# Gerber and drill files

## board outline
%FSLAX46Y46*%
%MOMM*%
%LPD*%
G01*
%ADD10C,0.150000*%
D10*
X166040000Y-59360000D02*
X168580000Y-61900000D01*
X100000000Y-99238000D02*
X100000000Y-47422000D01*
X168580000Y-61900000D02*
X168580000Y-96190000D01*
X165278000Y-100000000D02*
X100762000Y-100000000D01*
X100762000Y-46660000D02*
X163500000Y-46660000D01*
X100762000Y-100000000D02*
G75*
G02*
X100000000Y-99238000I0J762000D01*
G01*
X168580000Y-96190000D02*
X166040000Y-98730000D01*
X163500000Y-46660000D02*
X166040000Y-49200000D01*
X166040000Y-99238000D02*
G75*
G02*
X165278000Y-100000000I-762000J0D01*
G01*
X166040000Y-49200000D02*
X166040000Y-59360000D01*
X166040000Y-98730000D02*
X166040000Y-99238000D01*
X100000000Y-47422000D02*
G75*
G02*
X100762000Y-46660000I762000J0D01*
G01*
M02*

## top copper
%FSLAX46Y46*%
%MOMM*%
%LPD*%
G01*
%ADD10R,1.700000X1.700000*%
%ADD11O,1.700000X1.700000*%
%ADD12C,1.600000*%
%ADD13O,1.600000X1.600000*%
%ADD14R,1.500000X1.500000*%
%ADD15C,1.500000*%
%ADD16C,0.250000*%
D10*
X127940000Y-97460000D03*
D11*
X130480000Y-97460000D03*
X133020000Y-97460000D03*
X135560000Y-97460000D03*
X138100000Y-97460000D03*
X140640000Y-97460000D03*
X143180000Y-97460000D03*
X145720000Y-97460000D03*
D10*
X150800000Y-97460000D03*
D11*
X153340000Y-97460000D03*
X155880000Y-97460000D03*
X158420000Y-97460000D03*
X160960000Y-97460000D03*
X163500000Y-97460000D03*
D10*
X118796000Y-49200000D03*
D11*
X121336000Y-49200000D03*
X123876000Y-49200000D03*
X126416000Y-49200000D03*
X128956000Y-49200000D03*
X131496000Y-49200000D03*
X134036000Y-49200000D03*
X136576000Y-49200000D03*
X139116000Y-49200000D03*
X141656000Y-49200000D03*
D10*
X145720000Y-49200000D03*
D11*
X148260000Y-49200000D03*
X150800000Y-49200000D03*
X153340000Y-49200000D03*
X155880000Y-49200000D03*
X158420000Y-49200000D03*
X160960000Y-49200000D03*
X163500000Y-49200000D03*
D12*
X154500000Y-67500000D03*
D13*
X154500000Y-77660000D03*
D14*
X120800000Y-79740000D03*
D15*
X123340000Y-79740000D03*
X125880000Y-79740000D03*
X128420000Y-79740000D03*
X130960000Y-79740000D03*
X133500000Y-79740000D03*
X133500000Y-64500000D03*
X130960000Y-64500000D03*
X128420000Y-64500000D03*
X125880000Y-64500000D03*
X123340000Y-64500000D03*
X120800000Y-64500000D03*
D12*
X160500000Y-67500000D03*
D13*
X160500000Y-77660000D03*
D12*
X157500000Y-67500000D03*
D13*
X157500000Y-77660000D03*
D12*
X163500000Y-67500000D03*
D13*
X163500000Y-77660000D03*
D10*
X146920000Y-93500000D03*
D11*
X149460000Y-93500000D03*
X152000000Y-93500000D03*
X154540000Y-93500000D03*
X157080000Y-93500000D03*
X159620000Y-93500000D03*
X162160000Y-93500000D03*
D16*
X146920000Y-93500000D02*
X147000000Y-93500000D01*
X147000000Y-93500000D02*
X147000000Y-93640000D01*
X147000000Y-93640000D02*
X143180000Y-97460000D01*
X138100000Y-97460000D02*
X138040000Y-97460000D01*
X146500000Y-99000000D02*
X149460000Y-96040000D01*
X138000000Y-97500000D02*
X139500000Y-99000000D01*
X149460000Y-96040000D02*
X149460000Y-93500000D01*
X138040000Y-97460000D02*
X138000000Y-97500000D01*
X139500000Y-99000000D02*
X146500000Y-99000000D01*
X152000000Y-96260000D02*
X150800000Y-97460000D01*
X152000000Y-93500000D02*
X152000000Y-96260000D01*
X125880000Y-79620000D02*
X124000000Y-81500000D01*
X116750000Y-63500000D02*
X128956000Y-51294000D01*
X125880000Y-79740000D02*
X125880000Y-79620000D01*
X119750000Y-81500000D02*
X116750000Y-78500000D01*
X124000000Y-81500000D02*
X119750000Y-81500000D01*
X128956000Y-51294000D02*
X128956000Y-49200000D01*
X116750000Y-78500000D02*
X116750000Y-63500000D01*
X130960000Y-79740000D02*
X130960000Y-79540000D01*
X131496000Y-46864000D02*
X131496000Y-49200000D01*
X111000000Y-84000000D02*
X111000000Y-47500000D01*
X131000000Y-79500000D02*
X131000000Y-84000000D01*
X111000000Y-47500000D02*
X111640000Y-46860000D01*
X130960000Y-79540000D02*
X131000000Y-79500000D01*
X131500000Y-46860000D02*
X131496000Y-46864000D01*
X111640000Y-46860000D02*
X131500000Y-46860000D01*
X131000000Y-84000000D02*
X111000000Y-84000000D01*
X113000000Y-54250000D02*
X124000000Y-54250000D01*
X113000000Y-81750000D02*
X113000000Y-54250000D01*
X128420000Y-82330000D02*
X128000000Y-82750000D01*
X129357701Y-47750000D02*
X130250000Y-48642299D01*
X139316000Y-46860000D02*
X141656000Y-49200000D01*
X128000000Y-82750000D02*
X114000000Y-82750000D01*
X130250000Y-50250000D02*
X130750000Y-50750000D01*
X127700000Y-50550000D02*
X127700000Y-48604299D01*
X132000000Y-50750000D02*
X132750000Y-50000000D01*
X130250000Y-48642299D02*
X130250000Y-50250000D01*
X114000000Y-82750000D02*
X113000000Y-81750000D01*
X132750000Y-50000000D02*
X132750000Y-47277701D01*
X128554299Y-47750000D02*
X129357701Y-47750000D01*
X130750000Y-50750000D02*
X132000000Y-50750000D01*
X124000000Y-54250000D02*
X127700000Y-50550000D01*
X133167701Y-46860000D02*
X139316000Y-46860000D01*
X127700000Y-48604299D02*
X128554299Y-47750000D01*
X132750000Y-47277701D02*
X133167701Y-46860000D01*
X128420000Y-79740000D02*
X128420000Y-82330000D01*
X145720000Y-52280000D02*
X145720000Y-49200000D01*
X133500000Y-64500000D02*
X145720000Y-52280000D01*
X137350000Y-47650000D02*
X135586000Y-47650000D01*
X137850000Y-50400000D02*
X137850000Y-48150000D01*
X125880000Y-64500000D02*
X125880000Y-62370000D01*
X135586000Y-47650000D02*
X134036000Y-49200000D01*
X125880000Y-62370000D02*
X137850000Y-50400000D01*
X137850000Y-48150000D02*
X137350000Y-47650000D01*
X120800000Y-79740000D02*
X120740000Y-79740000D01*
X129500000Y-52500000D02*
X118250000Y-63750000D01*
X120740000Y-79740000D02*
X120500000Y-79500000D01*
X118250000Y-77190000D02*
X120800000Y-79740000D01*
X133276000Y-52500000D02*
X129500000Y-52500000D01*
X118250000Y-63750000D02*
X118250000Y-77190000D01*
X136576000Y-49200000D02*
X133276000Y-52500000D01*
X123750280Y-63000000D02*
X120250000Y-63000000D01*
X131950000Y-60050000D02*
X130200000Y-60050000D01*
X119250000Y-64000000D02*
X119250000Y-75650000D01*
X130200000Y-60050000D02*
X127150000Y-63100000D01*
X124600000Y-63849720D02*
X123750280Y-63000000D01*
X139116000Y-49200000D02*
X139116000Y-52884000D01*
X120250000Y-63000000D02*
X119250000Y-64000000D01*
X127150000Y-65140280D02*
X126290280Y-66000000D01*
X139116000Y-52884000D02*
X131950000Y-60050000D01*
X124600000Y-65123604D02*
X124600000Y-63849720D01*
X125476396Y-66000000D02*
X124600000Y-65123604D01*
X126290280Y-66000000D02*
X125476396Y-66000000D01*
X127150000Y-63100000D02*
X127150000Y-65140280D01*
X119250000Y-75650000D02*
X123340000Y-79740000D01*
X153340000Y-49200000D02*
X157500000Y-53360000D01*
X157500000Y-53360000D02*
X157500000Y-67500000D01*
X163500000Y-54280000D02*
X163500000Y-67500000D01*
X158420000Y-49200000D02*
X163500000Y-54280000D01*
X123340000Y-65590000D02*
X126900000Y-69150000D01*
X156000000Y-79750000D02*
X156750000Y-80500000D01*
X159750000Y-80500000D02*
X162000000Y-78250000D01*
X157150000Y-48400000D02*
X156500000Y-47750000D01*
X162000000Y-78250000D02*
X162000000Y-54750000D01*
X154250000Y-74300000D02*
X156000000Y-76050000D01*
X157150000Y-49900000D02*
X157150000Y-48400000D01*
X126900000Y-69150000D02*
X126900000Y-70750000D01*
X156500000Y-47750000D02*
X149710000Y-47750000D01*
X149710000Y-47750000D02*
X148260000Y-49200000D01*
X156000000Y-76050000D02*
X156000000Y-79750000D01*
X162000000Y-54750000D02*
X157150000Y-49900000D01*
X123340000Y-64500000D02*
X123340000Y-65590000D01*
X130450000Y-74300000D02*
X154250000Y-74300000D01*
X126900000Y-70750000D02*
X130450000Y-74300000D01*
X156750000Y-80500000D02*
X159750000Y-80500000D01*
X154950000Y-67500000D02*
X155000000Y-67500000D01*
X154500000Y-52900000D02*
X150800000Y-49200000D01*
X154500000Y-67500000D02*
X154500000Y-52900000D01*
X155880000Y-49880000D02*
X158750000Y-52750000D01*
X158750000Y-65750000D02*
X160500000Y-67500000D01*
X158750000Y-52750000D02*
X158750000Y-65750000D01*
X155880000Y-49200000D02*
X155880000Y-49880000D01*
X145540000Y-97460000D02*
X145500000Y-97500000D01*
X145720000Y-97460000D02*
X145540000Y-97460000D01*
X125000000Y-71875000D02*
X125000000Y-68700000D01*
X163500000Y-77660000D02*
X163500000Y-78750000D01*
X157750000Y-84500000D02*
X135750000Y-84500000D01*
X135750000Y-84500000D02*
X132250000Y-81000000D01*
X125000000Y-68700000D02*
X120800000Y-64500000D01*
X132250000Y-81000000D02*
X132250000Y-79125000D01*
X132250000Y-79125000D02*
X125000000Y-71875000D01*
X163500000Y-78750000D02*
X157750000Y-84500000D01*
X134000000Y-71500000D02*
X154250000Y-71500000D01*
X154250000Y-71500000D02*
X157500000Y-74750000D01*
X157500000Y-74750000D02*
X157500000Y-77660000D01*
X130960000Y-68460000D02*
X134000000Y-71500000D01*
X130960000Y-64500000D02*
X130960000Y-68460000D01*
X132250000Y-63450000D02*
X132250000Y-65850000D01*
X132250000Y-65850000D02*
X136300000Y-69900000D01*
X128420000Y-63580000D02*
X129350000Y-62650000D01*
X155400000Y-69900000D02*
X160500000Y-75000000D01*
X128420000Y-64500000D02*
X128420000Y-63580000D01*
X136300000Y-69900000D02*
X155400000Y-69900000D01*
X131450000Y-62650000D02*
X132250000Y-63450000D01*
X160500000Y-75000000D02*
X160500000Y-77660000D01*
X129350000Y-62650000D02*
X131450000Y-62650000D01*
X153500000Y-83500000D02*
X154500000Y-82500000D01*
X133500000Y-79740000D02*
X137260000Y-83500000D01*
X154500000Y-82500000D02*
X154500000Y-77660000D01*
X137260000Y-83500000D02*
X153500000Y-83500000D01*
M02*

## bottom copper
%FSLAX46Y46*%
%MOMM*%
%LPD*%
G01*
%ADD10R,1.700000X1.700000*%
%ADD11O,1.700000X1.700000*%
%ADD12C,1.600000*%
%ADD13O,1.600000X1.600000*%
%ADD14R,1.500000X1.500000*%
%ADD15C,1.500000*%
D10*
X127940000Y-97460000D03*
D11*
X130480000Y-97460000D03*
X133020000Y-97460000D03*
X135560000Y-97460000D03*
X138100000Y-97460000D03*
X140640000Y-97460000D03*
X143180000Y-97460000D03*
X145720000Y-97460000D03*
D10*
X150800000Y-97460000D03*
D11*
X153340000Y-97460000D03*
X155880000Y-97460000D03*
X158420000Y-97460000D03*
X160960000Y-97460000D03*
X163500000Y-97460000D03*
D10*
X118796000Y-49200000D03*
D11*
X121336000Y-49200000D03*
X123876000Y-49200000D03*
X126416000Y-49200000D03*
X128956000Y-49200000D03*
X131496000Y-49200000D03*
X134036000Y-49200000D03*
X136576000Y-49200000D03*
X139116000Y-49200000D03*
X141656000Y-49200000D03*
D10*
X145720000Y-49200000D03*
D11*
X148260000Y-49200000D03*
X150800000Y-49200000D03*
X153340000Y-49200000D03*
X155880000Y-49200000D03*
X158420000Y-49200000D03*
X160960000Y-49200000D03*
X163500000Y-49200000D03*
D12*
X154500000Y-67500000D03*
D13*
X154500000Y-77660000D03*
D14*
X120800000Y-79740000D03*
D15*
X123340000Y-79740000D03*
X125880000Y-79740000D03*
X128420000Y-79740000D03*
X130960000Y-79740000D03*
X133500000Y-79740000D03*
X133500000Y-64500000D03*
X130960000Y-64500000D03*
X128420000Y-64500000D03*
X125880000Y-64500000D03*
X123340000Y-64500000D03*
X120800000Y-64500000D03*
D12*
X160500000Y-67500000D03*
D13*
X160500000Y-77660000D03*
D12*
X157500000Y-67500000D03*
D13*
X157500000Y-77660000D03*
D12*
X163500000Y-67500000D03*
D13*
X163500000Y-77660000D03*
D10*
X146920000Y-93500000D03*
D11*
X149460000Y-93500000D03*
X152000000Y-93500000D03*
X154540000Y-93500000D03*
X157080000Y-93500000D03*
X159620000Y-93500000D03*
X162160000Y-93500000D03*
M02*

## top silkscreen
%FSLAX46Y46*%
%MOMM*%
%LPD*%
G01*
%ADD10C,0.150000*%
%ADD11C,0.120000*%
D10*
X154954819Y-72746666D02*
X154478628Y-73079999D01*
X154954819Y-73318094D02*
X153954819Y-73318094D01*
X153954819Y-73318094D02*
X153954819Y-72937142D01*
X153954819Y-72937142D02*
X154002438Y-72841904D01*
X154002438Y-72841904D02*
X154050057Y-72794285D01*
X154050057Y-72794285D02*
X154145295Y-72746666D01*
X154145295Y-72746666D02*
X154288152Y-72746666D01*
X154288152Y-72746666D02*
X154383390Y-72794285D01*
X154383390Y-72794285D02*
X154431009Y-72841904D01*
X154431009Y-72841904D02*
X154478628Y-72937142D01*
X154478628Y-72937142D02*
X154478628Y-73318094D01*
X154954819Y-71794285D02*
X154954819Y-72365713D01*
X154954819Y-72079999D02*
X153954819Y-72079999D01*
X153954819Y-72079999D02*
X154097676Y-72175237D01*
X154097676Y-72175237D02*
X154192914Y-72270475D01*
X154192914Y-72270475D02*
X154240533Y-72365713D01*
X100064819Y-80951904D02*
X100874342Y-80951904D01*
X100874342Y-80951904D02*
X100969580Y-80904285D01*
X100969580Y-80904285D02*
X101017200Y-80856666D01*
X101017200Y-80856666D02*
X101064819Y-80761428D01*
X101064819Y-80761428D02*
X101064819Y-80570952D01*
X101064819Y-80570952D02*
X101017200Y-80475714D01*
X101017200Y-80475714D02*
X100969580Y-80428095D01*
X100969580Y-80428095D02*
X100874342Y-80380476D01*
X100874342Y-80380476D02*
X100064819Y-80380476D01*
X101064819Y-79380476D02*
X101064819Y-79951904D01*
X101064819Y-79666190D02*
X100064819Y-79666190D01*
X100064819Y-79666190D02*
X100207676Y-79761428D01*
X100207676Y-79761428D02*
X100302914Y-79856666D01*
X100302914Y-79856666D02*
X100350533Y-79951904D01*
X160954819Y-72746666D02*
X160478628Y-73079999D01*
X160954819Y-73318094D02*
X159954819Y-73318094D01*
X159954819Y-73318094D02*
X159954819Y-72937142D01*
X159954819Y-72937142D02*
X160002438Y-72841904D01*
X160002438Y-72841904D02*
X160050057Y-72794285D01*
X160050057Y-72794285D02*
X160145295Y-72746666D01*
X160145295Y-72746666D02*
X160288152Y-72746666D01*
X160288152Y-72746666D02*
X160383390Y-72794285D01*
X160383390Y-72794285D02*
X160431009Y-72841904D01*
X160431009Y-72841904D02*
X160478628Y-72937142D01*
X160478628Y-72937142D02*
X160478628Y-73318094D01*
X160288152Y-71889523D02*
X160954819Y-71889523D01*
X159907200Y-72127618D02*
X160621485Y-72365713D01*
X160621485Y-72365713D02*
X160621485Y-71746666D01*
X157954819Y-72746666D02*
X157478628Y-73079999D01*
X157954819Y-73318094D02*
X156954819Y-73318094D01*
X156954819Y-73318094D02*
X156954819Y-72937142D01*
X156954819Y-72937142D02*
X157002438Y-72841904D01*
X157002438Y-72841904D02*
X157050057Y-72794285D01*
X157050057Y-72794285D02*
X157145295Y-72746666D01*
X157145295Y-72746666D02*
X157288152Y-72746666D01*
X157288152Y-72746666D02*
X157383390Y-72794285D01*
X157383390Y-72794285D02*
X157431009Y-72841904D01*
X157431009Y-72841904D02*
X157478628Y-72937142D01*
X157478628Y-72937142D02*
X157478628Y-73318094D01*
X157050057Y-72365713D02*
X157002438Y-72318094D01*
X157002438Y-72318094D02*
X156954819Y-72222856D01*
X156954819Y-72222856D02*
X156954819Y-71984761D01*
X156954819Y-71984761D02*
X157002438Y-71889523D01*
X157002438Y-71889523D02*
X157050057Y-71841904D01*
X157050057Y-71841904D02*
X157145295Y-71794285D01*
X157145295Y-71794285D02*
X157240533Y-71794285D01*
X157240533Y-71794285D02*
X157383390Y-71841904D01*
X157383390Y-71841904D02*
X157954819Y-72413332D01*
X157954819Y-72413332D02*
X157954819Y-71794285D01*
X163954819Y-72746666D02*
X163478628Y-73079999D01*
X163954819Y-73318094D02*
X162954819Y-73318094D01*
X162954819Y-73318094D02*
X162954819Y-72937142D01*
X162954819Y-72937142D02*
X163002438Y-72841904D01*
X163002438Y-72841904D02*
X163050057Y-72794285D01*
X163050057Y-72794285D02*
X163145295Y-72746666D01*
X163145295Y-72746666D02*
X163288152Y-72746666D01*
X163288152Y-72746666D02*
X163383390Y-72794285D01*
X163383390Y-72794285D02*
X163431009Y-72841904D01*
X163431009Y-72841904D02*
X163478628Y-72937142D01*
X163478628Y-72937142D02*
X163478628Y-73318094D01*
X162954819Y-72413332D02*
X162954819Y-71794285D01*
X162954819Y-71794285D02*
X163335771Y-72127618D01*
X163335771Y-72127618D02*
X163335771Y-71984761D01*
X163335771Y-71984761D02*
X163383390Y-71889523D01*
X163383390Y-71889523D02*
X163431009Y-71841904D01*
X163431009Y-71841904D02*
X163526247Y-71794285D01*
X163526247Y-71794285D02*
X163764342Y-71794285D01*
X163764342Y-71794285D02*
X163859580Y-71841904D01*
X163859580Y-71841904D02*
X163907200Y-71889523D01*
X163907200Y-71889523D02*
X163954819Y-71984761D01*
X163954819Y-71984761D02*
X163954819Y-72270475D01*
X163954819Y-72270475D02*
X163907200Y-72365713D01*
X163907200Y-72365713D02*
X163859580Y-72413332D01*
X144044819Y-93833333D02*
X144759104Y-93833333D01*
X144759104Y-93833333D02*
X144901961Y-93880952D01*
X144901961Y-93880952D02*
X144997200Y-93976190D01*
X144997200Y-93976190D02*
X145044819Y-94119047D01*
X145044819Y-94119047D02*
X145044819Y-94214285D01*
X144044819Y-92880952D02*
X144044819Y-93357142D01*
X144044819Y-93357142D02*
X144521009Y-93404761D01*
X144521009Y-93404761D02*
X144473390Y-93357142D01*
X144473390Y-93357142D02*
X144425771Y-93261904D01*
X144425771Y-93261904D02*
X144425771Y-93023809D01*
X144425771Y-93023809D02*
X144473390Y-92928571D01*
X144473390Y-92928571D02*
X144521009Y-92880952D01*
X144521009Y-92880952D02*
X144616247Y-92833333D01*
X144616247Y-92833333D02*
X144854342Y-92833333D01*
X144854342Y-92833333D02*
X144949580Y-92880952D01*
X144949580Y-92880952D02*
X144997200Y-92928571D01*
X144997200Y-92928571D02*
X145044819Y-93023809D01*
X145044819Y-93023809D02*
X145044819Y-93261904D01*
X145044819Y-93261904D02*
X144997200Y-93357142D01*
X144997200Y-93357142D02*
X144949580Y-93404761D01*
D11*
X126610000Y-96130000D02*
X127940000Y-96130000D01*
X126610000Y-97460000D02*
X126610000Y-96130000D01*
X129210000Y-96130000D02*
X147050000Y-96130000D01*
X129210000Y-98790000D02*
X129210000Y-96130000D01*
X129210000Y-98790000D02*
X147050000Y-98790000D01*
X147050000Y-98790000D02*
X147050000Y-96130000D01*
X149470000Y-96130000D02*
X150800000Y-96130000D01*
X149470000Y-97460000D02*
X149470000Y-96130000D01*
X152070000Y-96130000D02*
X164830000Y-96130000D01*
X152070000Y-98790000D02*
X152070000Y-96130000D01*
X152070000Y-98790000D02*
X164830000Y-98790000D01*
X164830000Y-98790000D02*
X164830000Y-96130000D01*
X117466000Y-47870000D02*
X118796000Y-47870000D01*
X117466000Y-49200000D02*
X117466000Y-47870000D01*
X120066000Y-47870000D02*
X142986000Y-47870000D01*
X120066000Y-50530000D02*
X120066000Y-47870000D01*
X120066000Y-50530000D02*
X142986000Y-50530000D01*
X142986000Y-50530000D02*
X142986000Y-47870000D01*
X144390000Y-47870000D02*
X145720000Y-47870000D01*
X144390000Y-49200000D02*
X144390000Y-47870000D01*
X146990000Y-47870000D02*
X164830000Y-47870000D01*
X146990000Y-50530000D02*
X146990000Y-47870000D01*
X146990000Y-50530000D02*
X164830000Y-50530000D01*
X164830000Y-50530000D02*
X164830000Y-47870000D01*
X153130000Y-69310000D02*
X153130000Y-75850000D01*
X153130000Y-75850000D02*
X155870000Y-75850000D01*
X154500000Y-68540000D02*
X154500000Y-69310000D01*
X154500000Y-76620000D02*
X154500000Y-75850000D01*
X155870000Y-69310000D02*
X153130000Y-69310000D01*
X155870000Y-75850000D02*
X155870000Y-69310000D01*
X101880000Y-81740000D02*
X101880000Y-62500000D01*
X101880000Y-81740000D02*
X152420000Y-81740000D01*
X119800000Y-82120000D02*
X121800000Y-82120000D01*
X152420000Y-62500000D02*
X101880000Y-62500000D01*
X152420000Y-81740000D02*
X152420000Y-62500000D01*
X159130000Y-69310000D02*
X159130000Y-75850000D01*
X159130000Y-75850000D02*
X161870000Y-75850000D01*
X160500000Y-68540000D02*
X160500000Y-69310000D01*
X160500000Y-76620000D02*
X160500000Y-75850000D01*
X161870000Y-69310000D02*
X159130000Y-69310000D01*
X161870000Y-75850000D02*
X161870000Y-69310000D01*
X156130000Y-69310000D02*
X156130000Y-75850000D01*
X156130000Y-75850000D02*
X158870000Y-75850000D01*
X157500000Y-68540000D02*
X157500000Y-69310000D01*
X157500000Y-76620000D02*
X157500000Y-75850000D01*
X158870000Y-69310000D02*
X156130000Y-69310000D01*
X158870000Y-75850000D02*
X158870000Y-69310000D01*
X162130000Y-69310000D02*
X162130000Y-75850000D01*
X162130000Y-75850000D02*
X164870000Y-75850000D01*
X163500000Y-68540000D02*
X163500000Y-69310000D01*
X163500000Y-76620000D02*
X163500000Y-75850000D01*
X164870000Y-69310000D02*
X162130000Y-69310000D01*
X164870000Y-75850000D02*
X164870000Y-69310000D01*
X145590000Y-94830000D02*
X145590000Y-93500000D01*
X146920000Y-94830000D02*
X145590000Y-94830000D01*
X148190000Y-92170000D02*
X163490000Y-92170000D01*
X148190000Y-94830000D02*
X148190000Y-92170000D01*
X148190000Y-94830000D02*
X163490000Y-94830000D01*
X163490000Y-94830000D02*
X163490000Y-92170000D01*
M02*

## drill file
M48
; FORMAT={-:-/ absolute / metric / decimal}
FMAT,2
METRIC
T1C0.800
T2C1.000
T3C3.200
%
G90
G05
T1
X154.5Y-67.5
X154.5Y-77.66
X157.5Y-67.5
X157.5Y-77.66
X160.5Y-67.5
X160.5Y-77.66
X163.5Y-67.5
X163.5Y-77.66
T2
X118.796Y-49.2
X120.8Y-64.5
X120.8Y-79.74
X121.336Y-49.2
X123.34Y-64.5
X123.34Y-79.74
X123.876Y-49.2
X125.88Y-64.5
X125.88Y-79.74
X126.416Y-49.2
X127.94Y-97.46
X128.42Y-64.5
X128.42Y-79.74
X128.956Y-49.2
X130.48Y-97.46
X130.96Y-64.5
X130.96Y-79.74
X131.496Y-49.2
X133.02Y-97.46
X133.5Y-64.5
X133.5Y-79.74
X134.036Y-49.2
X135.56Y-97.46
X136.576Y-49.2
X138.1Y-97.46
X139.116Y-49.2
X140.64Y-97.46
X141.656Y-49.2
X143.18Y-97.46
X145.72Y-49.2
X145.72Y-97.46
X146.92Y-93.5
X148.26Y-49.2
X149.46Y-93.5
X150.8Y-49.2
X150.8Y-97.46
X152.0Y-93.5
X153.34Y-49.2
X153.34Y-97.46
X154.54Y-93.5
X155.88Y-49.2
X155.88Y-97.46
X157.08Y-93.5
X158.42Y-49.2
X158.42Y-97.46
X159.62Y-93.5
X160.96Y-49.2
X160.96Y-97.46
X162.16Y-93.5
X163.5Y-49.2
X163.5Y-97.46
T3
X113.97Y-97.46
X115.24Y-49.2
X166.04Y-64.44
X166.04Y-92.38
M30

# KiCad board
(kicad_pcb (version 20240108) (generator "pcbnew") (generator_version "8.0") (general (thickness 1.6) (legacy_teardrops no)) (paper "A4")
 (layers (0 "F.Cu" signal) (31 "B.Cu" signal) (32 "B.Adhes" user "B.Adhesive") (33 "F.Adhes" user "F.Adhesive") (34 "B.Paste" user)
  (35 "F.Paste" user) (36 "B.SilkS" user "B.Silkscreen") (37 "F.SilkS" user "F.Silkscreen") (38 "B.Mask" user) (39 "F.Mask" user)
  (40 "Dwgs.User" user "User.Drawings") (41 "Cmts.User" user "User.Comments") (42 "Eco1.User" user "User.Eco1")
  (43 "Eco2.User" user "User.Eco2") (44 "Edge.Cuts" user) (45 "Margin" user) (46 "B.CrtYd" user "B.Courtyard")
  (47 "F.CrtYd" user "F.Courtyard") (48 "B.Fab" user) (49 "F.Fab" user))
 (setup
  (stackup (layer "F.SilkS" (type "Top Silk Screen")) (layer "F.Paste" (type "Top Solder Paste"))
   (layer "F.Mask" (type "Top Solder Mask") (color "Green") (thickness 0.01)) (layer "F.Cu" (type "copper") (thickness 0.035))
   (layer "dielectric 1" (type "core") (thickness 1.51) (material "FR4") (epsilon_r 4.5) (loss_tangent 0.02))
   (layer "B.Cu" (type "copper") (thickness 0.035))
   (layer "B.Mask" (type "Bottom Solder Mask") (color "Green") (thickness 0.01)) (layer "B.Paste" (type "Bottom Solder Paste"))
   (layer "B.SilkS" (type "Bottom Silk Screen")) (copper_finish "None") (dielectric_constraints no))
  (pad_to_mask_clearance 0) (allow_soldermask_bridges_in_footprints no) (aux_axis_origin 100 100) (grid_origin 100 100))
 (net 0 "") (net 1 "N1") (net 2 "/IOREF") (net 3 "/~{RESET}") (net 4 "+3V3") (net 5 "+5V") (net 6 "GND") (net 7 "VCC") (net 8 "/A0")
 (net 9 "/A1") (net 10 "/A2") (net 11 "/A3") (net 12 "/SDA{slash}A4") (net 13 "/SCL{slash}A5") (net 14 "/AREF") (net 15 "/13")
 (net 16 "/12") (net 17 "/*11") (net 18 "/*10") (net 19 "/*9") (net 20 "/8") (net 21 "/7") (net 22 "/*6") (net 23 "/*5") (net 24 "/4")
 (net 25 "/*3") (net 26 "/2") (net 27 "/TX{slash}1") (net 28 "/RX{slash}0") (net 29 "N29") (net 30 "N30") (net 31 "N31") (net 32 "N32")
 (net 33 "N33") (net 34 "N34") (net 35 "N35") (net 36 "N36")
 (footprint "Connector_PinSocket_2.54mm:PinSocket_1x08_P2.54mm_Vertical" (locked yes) (layer "F.Cu") (at 127.94 97.46 90)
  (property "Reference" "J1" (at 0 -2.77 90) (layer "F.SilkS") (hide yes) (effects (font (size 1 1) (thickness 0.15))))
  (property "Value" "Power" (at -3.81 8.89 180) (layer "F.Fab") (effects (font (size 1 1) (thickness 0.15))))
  (fp_line (start 1.33 -1.33) (end 1.33 0) (stroke (width 0.12) (type solid)) (layer "F.SilkS"))
  (fp_line (start 0 -1.33) (end 1.33 -1.33) (stroke (width 0.12) (type solid)) (layer "F.SilkS"))
  (fp_line (start 1.33 1.27) (end 1.33 19.11) (stroke (width 0.12) (type solid)) (layer "F.SilkS"))
  (fp_line (start -1.33 1.27) (end 1.33 1.27) (stroke (width 0.12) (type solid)) (layer "F.SilkS"))
  (fp_line (start -1.33 1.27) (end -1.33 19.11) (stroke (width 0.12) (type solid)) (layer "F.SilkS"))
  (fp_line (start -1.33 19.11) (end 1.33 19.11) (stroke (width 0.12) (type solid)) (layer "F.SilkS"))
  (pad "1" thru_hole rect (at 0 0 90) (size 1.7 1.7) (drill 1) (layers "*.Cu" "*.Mask") (remove_unused_layers no) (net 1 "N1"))
  (pad "2" thru_hole oval (at 0 2.54 90) (size 1.7 1.7) (drill 1) (layers "*.Cu" "*.Mask") (remove_unused_layers no) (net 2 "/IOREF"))
  (pad "3" thru_hole oval (at 0 5.08 90) (size 1.7 1.7) (drill 1) (layers "*.Cu" "*.Mask") (remove_unused_layers no) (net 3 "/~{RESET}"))
  (pad "4" thru_hole oval (at 0 7.62 90) (size 1.7 1.7) (drill 1) (layers "*.Cu" "*.Mask") (remove_unused_layers no) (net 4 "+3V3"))
  (pad "5" thru_hole oval (at 0 10.16 90) (size 1.7 1.7) (drill 1) (layers "*.Cu" "*.Mask") (remove_unused_layers no) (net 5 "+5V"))
  (pad "6" thru_hole oval (at 0 12.7 90) (size 1.7 1.7) (drill 1) (layers "*.Cu" "*.Mask") (remove_unused_layers no) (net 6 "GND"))
  (pad "7" thru_hole oval (at 0 15.24 90) (size 1.7 1.7) (drill 1) (layers "*.Cu" "*.Mask") (remove_unused_layers no) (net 6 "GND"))
  (pad "8" thru_hole oval (at 0 17.78 90) (size 1.7 1.7) (drill 1) (layers "*.Cu" "*.Mask") (remove_unused_layers no) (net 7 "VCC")))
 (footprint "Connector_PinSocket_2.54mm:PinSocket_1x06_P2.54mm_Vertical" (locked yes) (layer "F.Cu") (at 150.8 97.46 90)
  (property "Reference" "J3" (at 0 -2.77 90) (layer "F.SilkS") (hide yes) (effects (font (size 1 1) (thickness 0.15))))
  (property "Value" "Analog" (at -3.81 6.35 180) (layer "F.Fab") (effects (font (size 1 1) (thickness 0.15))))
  (fp_line (start 1.33 -1.33) (end 1.33 0) (stroke (width 0.12) (type solid)) (layer "F.SilkS"))
  (fp_line (start 0 -1.33) (end 1.33 -1.33) (stroke (width 0.12) (type solid)) (layer "F.SilkS"))
  (fp_line (start 1.33 1.27) (end 1.33 14.03) (stroke (width 0.12) (type solid)) (layer "F.SilkS"))
  (fp_line (start -1.33 1.27) (end 1.33 1.27) (stroke (width 0.12) (type solid)) (layer "F.SilkS"))
  (fp_line (start -1.33 1.27) (end -1.33 14.03) (stroke (width 0.12) (type solid)) (layer "F.SilkS"))
  (fp_line (start -1.33 14.03) (end 1.33 14.03) (stroke (width 0.12) (type solid)) (layer "F.SilkS"))
  (pad "1" thru_hole rect (at 0 0 90) (size 1.7 1.7) (drill 1) (layers "*.Cu" "*.Mask") (remove_unused_layers no) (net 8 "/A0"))
  (pad "2" thru_hole oval (at 0 2.54 90) (size 1.7 1.7) (drill 1) (layers "*.Cu" "*.Mask") (remove_unused_layers no) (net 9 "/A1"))
  (pad "3" thru_hole oval (at 0 5.08 90) (size 1.7 1.7) (drill 1) (layers "*.Cu" "*.Mask") (remove_unused_layers no) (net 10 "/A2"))
  (pad "4" thru_hole oval (at 0 7.62 90) (size 1.7 1.7) (drill 1) (layers "*.Cu" "*.Mask") (remove_unused_layers no) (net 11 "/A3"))
  (pad "5" thru_hole oval (at 0 10.16 90) (size 1.7 1.7) (drill 1) (layers "*.Cu" "*.Mask") (remove_unused_layers no)
   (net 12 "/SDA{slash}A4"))
  (pad "6" thru_hole oval (at 0 12.7 90) (size 1.7 1.7) (drill 1) (layers "*.Cu" "*.Mask") (remove_unused_layers no)
   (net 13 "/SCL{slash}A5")))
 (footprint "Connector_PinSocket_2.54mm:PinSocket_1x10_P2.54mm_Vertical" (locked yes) (layer "F.Cu") (at 118.796 49.2 90)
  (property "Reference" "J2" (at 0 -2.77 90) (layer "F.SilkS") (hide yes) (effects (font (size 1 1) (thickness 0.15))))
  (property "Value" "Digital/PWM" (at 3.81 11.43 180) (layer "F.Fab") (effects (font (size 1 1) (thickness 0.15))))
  (fp_line (start 1.33 -1.33) (end 1.33 0) (stroke (width 0.12) (type solid)) (layer "F.SilkS"))
  (fp_line (start 0 -1.33) (end 1.33 -1.33) (stroke (width 0.12) (type solid)) (layer "F.SilkS"))
  (fp_line (start 1.33 1.27) (end 1.33 24.19) (stroke (width 0.12) (type solid)) (layer "F.SilkS"))
  (fp_line (start -1.33 1.27) (end 1.33 1.27) (stroke (width 0.12) (type solid)) (layer "F.SilkS"))
  (fp_line (start -1.33 1.27) (end -1.33 24.19) (stroke (width 0.12) (type solid)) (layer "F.SilkS"))
  (fp_line (start -1.33 24.19) (end 1.33 24.19) (stroke (width 0.12) (type solid)) (layer "F.SilkS"))
  (pad "1" thru_hole rect (at 0 0 90) (size 1.7 1.7) (drill 1) (layers "*.Cu" "*.Mask") (remove_unused_layers no) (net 13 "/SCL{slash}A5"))
  (pad "2" thru_hole oval (at 0 2.54 90) (size 1.7 1.7) (drill 1) (layers "*.Cu" "*.Mask") (remove_unused_layers no)
   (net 12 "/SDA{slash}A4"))
  (pad "3" thru_hole oval (at 0 5.08 90) (size 1.7 1.7) (drill 1) (layers "*.Cu" "*.Mask") (remove_unused_layers no) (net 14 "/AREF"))
  (pad "4" thru_hole oval (at 0 7.62 90) (size 1.7 1.7) (drill 1) (layers "*.Cu" "*.Mask") (remove_unused_layers no) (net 6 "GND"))
  (pad "5" thru_hole oval (at 0 10.16 90) (size 1.7 1.7) (drill 1) (layers "*.Cu" "*.Mask") (remove_unused_layers no) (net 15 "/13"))
  (pad "6" thru_hole oval (at 0 12.7 90) (size 1.7 1.7) (drill 1) (layers "*.Cu" "*.Mask") (remove_unused_layers no) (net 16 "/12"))
  (pad "7" thru_hole oval (at 0 15.24 90) (size 1.7 1.7) (drill 1) (layers "*.Cu" "*.Mask") (remove_unused_layers no) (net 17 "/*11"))
  (pad "8" thru_hole oval (at 0 17.78 90) (size 1.7 1.7) (drill 1) (layers "*.Cu" "*.Mask") (remove_unused_layers no) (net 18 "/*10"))
  (pad "9" thru_hole oval (at 0 20.32 90) (size 1.7 1.7) (drill 1) (layers "*.Cu" "*.Mask") (remove_unused_layers no) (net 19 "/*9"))
  (pad "10" thru_hole oval (at 0 22.86 90) (size 1.7 1.7) (drill 1) (layers "*.Cu" "*.Mask") (remove_unused_layers no) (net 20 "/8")))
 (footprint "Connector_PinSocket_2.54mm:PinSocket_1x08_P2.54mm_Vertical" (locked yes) (layer "F.Cu") (at 145.72 49.2 90)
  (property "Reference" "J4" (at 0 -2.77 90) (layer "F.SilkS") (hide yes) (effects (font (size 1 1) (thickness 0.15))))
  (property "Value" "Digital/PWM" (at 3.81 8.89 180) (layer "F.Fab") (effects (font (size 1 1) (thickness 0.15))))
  (fp_line (start 1.33 -1.33) (end 1.33 0) (stroke (width 0.12) (type solid)) (layer "F.SilkS"))
  (fp_line (start 0 -1.33) (end 1.33 -1.33) (stroke (width 0.12) (type solid)) (layer "F.SilkS"))
  (fp_line (start 1.33 1.27) (end 1.33 19.11) (stroke (width 0.12) (type solid)) (layer "F.SilkS"))
  (fp_line (start -1.33 1.27) (end 1.33 1.27) (stroke (width 0.12) (type solid)) (layer "F.SilkS"))
  (fp_line (start -1.33 1.27) (end -1.33 19.11) (stroke (width 0.12) (type solid)) (layer "F.SilkS"))
  (fp_line (start -1.33 19.11) (end 1.33 19.11) (stroke (width 0.12) (type solid)) (layer "F.SilkS"))
  (pad "1" thru_hole rect (at 0 0 90) (size 1.7 1.7) (drill 1) (layers "*.Cu" "*.Mask") (remove_unused_layers no) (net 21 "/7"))
  (pad "2" thru_hole oval (at 0 2.54 90) (size 1.7 1.7) (drill 1) (layers "*.Cu" "*.Mask") (remove_unused_layers no) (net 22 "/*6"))
  (pad "3" thru_hole oval (at 0 5.08 90) (size 1.7 1.7) (drill 1) (layers "*.Cu" "*.Mask") (remove_unused_layers no) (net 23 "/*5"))
  (pad "4" thru_hole oval (at 0 7.62 90) (size 1.7 1.7) (drill 1) (layers "*.Cu" "*.Mask") (remove_unused_layers no) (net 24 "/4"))
  (pad "5" thru_hole oval (at 0 10.16 90) (size 1.7 1.7) (drill 1) (layers "*.Cu" "*.Mask") (remove_unused_layers no) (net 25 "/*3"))
  (pad "6" thru_hole oval (at 0 12.7 90) (size 1.7 1.7) (drill 1) (layers "*.Cu" "*.Mask") (remove_unused_layers no) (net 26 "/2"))
  (pad "7" thru_hole oval (at 0 15.24 90) (size 1.7 1.7) (drill 1) (layers "*.Cu" "*.Mask") (remove_unused_layers no) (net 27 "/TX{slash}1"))
  (pad "8" thru_hole oval (at 0 17.78 90) (size 1.7 1.7) (drill 1) (layers "*.Cu" "*.Mask") (remove_unused_layers no) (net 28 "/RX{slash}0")))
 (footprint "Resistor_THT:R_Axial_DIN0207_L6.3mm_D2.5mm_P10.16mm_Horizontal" (layer "F.Cu") (at 154.5 67.5 -90)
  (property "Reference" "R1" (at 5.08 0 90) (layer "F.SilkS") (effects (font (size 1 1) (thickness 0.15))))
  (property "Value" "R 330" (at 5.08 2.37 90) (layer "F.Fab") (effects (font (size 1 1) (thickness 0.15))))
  (fp_line (start 1.81 1.37) (end 8.35 1.37) (stroke (width 0.12) (type solid)) (layer "F.SilkS"))
  (fp_line (start 8.35 1.37) (end 8.35 -1.37) (stroke (width 0.12) (type solid)) (layer "F.SilkS"))
  (fp_line (start 1.04 0) (end 1.81 0) (stroke (width 0.12) (type solid)) (layer "F.SilkS"))
  (fp_line (start 9.12 0) (end 8.35 0) (stroke (width 0.12) (type solid)) (layer "F.SilkS"))
  (fp_line (start 1.81 -1.37) (end 1.81 1.37) (stroke (width 0.12) (type solid)) (layer "F.SilkS"))
  (fp_line (start 8.35 -1.37) (end 1.81 -1.37) (stroke (width 0.12) (type solid)) (layer "F.SilkS"))
  (pad "1" thru_hole circle (at 0 0 270) (size 1.6 1.6) (drill 0.8) (layers "*.Cu" "*.Mask") (remove_unused_layers no) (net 23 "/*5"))
  (pad "2" thru_hole oval (at 10.16 0 270) (size 1.6 1.6) (drill 0.8) (layers "*.Cu" "*.Mask") (remove_unused_layers no) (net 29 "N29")))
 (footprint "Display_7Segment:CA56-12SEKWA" (layer "F.Cu") (at 120.8 79.74 90)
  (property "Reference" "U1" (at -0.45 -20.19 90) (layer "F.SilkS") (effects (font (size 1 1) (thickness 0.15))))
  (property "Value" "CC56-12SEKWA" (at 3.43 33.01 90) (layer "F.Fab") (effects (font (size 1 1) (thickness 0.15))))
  (fp_line (start -2 -18.92) (end 17.24 -18.92) (stroke (width 0.12) (type solid)) (layer "F.SilkS"))
  (fp_line (start -2 -18.92) (end -2 31.62) (stroke (width 0.12) (type solid)) (layer "F.SilkS"))
  (fp_line (start -2.38 -1) (end -2.38 1) (stroke (width 0.12) (type solid)) (layer "F.SilkS"))
  (fp_line (start 17.24 31.62) (end 17.24 -18.92) (stroke (width 0.12) (type solid)) (layer "F.SilkS"))
  (fp_line (start -2 31.62) (end 17.24 31.62) (stroke (width 0.12) (type solid)) (layer "F.SilkS"))
  (pad "1" thru_hole rect (at 0 0 90) (size 1.5 1.5) (drill 1) (layers "*.Cu" "*.Mask") (remove_unused_layers no) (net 18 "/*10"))
  (pad "2" thru_hole circle (at 0 2.54 90) (size 1.5 1.5) (drill 1) (layers "*.Cu" "*.Mask") (remove_unused_layers no) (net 19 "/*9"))
  (pad "3" thru_hole circle (at 0 5.08 90) (size 1.5 1.5) (drill 1) (layers "*.Cu" "*.Mask") (remove_unused_layers no) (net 15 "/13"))
  (pad "4" thru_hole circle (at 0 7.62 90) (size 1.5 1.5) (drill 1) (layers "*.Cu" "*.Mask") (remove_unused_layers no) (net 20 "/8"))
  (pad "5" thru_hole circle (at 0 10.16 90) (size 1.5 1.5) (drill 1) (layers "*.Cu" "*.Mask") (remove_unused_layers no) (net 16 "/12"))
  (pad "6" thru_hole circle (at 0 12.7 90) (size 1.5 1.5) (drill 1) (layers "*.Cu" "*.Mask") (remove_unused_layers no) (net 29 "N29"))
  (pad "7" thru_hole circle (at 15.24 12.7 90) (size 1.5 1.5) (drill 1) (layers "*.Cu" "*.Mask") (remove_unused_layers no) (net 21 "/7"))
  (pad "8" thru_hole circle (at 15.24 10.16 90) (size 1.5 1.5) (drill 1) (layers "*.Cu" "*.Mask") (remove_unused_layers no) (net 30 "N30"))
  (pad "9" thru_hole circle (at 15.24 7.62 90) (size 1.5 1.5) (drill 1) (layers "*.Cu" "*.Mask") (remove_unused_layers no) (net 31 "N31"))
  (pad "10" thru_hole circle (at 15.24 5.08 90) (size 1.5 1.5) (drill 1) (layers "*.Cu" "*.Mask") (remove_unused_layers no) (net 17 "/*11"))
  (pad "11" thru_hole circle (at 15.24 2.54 90) (size 1.5 1.5) (drill 1) (layers "*.Cu" "*.Mask") (remove_unused_layers no) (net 22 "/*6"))
  (pad "12" thru_hole circle (at 15.24 0 90) (size 1.5 1.5) (drill 1) (layers "*.Cu" "*.Mask") (remove_unused_layers no) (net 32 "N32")))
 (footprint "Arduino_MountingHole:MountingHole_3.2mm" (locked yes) (layer "F.Cu") (at 115.24 49.2)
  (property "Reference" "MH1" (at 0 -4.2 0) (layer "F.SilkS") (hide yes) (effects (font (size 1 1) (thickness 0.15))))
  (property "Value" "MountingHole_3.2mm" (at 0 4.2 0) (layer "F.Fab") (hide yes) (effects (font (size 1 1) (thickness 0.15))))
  (pad "" np_thru_hole circle (at 0 0) (size 3.2 3.2) (drill 3.2) (layers "*.Cu" "*.Mask")))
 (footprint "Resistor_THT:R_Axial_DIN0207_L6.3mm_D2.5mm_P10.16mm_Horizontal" (layer "F.Cu") (at 160.5 67.5 -90)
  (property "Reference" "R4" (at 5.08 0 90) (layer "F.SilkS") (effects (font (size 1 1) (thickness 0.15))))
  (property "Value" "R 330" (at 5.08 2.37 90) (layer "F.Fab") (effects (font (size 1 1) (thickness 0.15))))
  (fp_line (start 1.81 1.37) (end 8.35 1.37) (stroke (width 0.12) (type solid)) (layer "F.SilkS"))
  (fp_line (start 8.35 1.37) (end 8.35 -1.37) (stroke (width 0.12) (type solid)) (layer "F.SilkS"))
  (fp_line (start 1.04 0) (end 1.81 0) (stroke (width 0.12) (type solid)) (layer "F.SilkS"))
  (fp_line (start 9.12 0) (end 8.35 0) (stroke (width 0.12) (type solid)) (layer "F.SilkS"))
  (fp_line (start 1.81 -1.37) (end 1.81 1.37) (stroke (width 0.12) (type solid)) (layer "F.SilkS"))
  (fp_line (start 8.35 -1.37) (end 1.81 -1.37) (stroke (width 0.12) (type solid)) (layer "F.SilkS"))
  (pad "1" thru_hole circle (at 0 0 270) (size 1.6 1.6) (drill 0.8) (layers "*.Cu" "*.Mask") (remove_unused_layers no) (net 25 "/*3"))
  (pad "2" thru_hole oval (at 10.16 0 270) (size 1.6 1.6) (drill 0.8) (layers "*.Cu" "*.Mask") (remove_unused_layers no) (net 31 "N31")))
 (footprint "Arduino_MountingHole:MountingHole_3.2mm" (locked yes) (layer "F.Cu") (at 113.97 97.46)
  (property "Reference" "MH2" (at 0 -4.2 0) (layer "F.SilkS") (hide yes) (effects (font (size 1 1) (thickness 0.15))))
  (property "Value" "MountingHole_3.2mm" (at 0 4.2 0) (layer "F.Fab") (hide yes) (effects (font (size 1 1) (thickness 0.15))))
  (pad "" np_thru_hole circle (at 0 0) (size 3.2 3.2) (drill 3.2) (layers "*.Cu" "*.Mask")))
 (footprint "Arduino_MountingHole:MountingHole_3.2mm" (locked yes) (layer "F.Cu") (at 166.04 64.44)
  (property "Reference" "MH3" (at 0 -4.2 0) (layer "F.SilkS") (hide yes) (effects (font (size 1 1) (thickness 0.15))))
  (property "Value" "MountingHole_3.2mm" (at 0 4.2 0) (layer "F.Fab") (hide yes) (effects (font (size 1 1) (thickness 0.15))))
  (pad "" np_thru_hole circle (at 0 0) (size 3.2 3.2) (drill 3.2) (layers "*.Cu" "*.Mask")))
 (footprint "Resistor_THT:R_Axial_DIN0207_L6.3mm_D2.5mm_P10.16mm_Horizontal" (layer "F.Cu") (at 157.5 67.5 -90)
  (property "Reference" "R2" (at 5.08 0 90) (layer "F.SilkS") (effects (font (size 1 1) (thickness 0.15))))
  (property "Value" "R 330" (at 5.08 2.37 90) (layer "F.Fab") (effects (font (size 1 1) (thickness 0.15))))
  (fp_line (start 1.81 1.37) (end 8.35 1.37) (stroke (width 0.12) (type solid)) (layer "F.SilkS"))
  (fp_line (start 8.35 1.37) (end 8.35 -1.37) (stroke (width 0.12) (type solid)) (layer "F.SilkS"))
  (fp_line (start 1.04 0) (end 1.81 0) (stroke (width 0.12) (type solid)) (layer "F.SilkS"))
  (fp_line (start 9.12 0) (end 8.35 0) (stroke (width 0.12) (type solid)) (layer "F.SilkS"))
  (fp_line (start 1.81 -1.37) (end 1.81 1.37) (stroke (width 0.12) (type solid)) (layer "F.SilkS"))
  (fp_line (start 8.35 -1.37) (end 1.81 -1.37) (stroke (width 0.12) (type solid)) (layer "F.SilkS"))
  (pad "1" thru_hole circle (at 0 0 270) (size 1.6 1.6) (drill 0.8) (layers "*.Cu" "*.Mask") (remove_unused_layers no) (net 24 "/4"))
  (pad "2" thru_hole oval (at 10.16 0 270) (size 1.6 1.6) (drill 0.8) (layers "*.Cu" "*.Mask") (remove_unused_layers no) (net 30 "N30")))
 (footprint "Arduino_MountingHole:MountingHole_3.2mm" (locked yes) (layer "F.Cu") (at 166.04 92.38)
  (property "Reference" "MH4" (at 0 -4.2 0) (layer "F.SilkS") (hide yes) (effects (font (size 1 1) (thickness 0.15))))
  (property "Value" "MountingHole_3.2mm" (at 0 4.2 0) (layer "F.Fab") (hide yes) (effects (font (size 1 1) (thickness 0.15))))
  (pad "" np_thru_hole circle (at 0 0) (size 3.2 3.2) (drill 3.2) (layers "*.Cu" "*.Mask")))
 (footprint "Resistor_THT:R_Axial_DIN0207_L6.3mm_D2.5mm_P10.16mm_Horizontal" (layer "F.Cu") (at 163.5 67.5 -90)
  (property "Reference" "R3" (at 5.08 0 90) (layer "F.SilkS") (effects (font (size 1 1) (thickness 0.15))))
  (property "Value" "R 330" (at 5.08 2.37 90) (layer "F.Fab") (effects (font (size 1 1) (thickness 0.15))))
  (fp_line (start 1.81 1.37) (end 8.35 1.37) (stroke (width 0.12) (type solid)) (layer "F.SilkS"))
  (fp_line (start 8.35 1.37) (end 8.35 -1.37) (stroke (width 0.12) (type solid)) (layer "F.SilkS"))
  (fp_line (start 1.04 0) (end 1.81 0) (stroke (width 0.12) (type solid)) (layer "F.SilkS"))
  (fp_line (start 9.12 0) (end 8.35 0) (stroke (width 0.12) (type solid)) (layer "F.SilkS"))
  (fp_line (start 1.81 -1.37) (end 1.81 1.37) (stroke (width 0.12) (type solid)) (layer "F.SilkS"))
  (fp_line (start 8.35 -1.37) (end 1.81 -1.37) (stroke (width 0.12) (type solid)) (layer "F.SilkS"))
  (pad "1" thru_hole circle (at 0 0 270) (size 1.6 1.6) (drill 0.8) (layers "*.Cu" "*.Mask") (remove_unused_layers no) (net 26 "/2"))
  (pad "2" thru_hole oval (at 10.16 0 270) (size 1.6 1.6) (drill 0.8) (layers "*.Cu" "*.Mask") (remove_unused_layers no) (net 32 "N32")))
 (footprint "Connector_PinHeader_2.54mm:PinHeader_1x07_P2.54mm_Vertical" (layer "F.Cu") (at 146.92 93.5 90)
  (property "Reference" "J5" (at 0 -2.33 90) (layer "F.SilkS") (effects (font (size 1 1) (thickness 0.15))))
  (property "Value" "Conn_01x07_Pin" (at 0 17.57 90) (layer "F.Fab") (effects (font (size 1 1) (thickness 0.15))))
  (fp_line (start -1.33 -1.33) (end 0 -1.33) (stroke (width 0.12) (type solid)) (layer "F.SilkS"))
  (fp_line (start -1.33 0) (end -1.33 -1.33) (stroke (width 0.12) (type solid)) (layer "F.SilkS"))
  (fp_line (start 1.33 1.27) (end 1.33 16.57) (stroke (width 0.12) (type solid)) (layer "F.SilkS"))
  (fp_line (start -1.33 1.27) (end 1.33 1.27) (stroke (width 0.12) (type solid)) (layer "F.SilkS"))
  (fp_line (start -1.33 1.27) (end -1.33 16.57) (stroke (width 0.12) (type solid)) (layer "F.SilkS"))
  (fp_line (start -1.33 16.57) (end 1.33 16.57) (stroke (width 0.12) (type solid)) (layer "F.SilkS"))
  (pad "1" thru_hole rect (at 0 0 90) (size 1.7 1.7) (drill 1) (layers "*.Cu" "*.Mask") (remove_unused_layers no) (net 6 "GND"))
  (pad "2" thru_hole oval (at 0 2.54 90) (size 1.7 1.7) (drill 1) (layers "*.Cu" "*.Mask") (remove_unused_layers no) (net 5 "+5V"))
  (pad "3" thru_hole oval (at 0 5.08 90) (size 1.7 1.7) (drill 1) (layers "*.Cu" "*.Mask") (remove_unused_layers no) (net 8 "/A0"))
  (pad "4" thru_hole oval (at 0 7.62 90) (size 1.7 1.7) (drill 1) (layers "*.Cu" "*.Mask") (remove_unused_layers no) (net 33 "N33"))
  (pad "5" thru_hole oval (at 0 10.16 90) (size 1.7 1.7) (drill 1) (layers "*.Cu" "*.Mask") (remove_unused_layers no) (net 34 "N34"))
  (pad "6" thru_hole oval (at 0 12.7 90) (size 1.7 1.7) (drill 1) (layers "*.Cu" "*.Mask") (remove_unused_layers no) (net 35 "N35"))
  (pad "7" thru_hole oval (at 0 15.24 90) (size 1.7 1.7) (drill 1) (layers "*.Cu" "*.Mask") (remove_unused_layers no) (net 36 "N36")))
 (gr_line (start 166.04 59.36) (end 168.58 61.9) (stroke (width 0.15) (type solid)) (layer "Edge.Cuts"))
 (gr_line (start 100 99.238) (end 100 47.422) (stroke (width 0.15) (type solid)) (layer "Edge.Cuts"))
 (gr_line (start 168.58 61.9) (end 168.58 96.19) (stroke (width 0.15) (type solid)) (layer "Edge.Cuts"))
 (gr_line (start 165.278 100) (end 100.762 100) (stroke (width 0.15) (type solid)) (layer "Edge.Cuts"))
 (gr_line (start 100.762 46.66) (end 163.5 46.66) (stroke (width 0.15) (type solid)) (layer "Edge.Cuts"))
 (gr_arc (start 100.762 100) (mid 100.223185 99.776815) (end 100 99.238) (stroke (width 0.15) (type solid)) (layer "Edge.Cuts"))
 (gr_line (start 168.58 96.19) (end 166.04 98.73) (stroke (width 0.15) (type solid)) (layer "Edge.Cuts"))
 (gr_line (start 163.5 46.66) (end 166.04 49.2) (stroke (width 0.15) (type solid)) (layer "Edge.Cuts"))
 (gr_arc (start 166.04 99.238) (mid 165.816815 99.776815) (end 165.278 100) (stroke (width 0.15) (type solid)) (layer "Edge.Cuts"))
 (gr_line (start 166.04 49.2) (end 166.04 59.36) (stroke (width 0.15) (type solid)) (layer "Edge.Cuts"))
 (gr_line (start 166.04 98.73) (end 166.04 99.238) (stroke (width 0.15) (type solid)) (layer "Edge.Cuts"))
 (gr_arc (start 100 47.422) (mid 100.223185 46.883185) (end 100.762 46.66) (stroke (width 0.15) (type solid)) (layer "Edge.Cuts"))
 (segment (start 146.92 93.5) (end 147 93.5) (width 0.25) (layer "F.Cu") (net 6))
 (segment (start 147 93.5) (end 147 93.64) (width 0.25) (layer "F.Cu") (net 6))
 (segment (start 147 93.64) (end 143.18 97.46) (width 0.25) (layer "F.Cu") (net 6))
 (segment (start 138.1 97.46) (end 138.04 97.46) (width 0.25) (layer "F.Cu") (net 5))
 (segment (start 146.5 99) (end 149.46 96.04) (width 0.25) (layer "F.Cu") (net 5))
 (segment (start 138 97.5) (end 139.5 99) (width 0.25) (layer "F.Cu") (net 5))
 (segment (start 149.46 96.04) (end 149.46 93.5) (width 0.25) (layer "F.Cu") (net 5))
 (segment (start 138.04 97.46) (end 138 97.5) (width 0.25) (layer "F.Cu") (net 5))
 (segment (start 139.5 99) (end 146.5 99) (width 0.25) (layer "F.Cu") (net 5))
 (segment (start 152 96.26) (end 150.8 97.46) (width 0.25) (layer "F.Cu") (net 8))
 (segment (start 152 93.5) (end 152 96.26) (width 0.25) (layer "F.Cu") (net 8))
 (segment (start 125.88 79.62) (end 124 81.5) (width 0.25) (layer "F.Cu") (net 15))
 (segment (start 116.75 63.5) (end 128.956 51.294) (width 0.25) (layer "F.Cu") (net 15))
 (segment (start 125.88 79.74) (end 125.88 79.62) (width 0.25) (layer "F.Cu") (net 15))
 (segment (start 119.75 81.5) (end 116.75 78.5) (width 0.25) (layer "F.Cu") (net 15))
 (segment (start 124 81.5) (end 119.75 81.5) (width 0.25) (layer "F.Cu") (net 15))
 (segment (start 128.956 51.294) (end 128.956 49.2) (width 0.25) (layer "F.Cu") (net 15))
 (segment (start 116.75 78.5) (end 116.75 63.5) (width 0.25) (layer "F.Cu") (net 15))
 (segment (start 130.96 79.74) (end 130.96 79.54) (width 0.25) (layer "F.Cu") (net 16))
 (segment (start 131.496 46.864) (end 131.496 49.2) (width 0.25) (layer "F.Cu") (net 16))
 (segment (start 111 84) (end 111 47.5) (width 0.25) (layer "F.Cu") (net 16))
 (segment (start 131 79.5) (end 131 84) (width 0.25) (layer "F.Cu") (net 16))
 (segment (start 111 47.5) (end 111.64 46.86) (width 0.25) (layer "F.Cu") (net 16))
 (segment (start 130.96 79.54) (end 131 79.5) (width 0.25) (layer "F.Cu") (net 16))
 (segment (start 131.5 46.86) (end 131.496 46.864) (width 0.25) (layer "F.Cu") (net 16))
 (segment (start 111.64 46.86) (end 131.5 46.86) (width 0.25) (layer "F.Cu") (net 16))
 (segment (start 131 84) (end 111 84) (width 0.25) (layer "F.Cu") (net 16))
 (segment (start 113 54.25) (end 124 54.25) (width 0.25) (layer "F.Cu") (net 20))
 (segment (start 113 81.75) (end 113 54.25) (width 0.25) (layer "F.Cu") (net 20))
 (segment (start 128.42 82.33) (end 128 82.75) (width 0.25) (layer "F.Cu") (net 20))
 (segment (start 129.357701 47.75) (end 130.25 48.642299) (width 0.25) (layer "F.Cu") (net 20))
 (segment (start 139.316 46.86) (end 141.656 49.2) (width 0.25) (layer "F.Cu") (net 20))
 (segment (start 128 82.75) (end 114 82.75) (width 0.25) (layer "F.Cu") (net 20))
 (segment (start 130.25 50.25) (end 130.75 50.75) (width 0.25) (layer "F.Cu") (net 20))
 (segment (start 127.7 50.55) (end 127.7 48.604299) (width 0.25) (layer "F.Cu") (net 20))
 (segment (start 132 50.75) (end 132.75 50) (width 0.25) (layer "F.Cu") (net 20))
 (segment (start 130.25 48.642299) (end 130.25 50.25) (width 0.25) (layer "F.Cu") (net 20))
 (segment (start 114 82.75) (end 113 81.75) (width 0.25) (layer "F.Cu") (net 20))
 (segment (start 132.75 50) (end 132.75 47.277701) (width 0.25) (layer "F.Cu") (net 20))
 (segment (start 128.554299 47.75) (end 129.357701 47.75) (width 0.25) (layer "F.Cu") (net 20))
 (segment (start 130.75 50.75) (end 132 50.75) (width 0.25) (layer "F.Cu") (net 20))
 (segment (start 124 54.25) (end 127.7 50.55) (width 0.25) (layer "F.Cu") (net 20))
 (segment (start 133.167701 46.86) (end 139.316 46.86) (width 0.25) (layer "F.Cu") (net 20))
 (segment (start 127.7 48.604299) (end 128.554299 47.75) (width 0.25) (layer "F.Cu") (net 20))
 (segment (start 132.75 47.277701) (end 133.167701 46.86) (width 0.25) (layer "F.Cu") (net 20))
 (segment (start 128.42 79.74) (end 128.42 82.33) (width 0.25) (layer "F.Cu") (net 20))
 (segment (start 145.72 52.28) (end 145.72 49.2) (width 0.25) (layer "F.Cu") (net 21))
 (segment (start 133.5 64.5) (end 145.72 52.28) (width 0.25) (layer "F.Cu") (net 21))
 (segment (start 137.35 47.65) (end 135.586 47.65) (width 0.25) (layer "F.Cu") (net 17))
 (segment (start 137.85 50.4) (end 137.85 48.15) (width 0.25) (layer "F.Cu") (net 17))
 (segment (start 125.88 64.5) (end 125.88 62.37) (width 0.25) (layer "F.Cu") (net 17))
 (segment (start 135.586 47.65) (end 134.036 49.2) (width 0.25) (layer "F.Cu") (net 17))
 (segment (start 125.88 62.37) (end 137.85 50.4) (width 0.25) (layer "F.Cu") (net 17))
 (segment (start 137.85 48.15) (end 137.35 47.65) (width 0.25) (layer "F.Cu") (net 17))
 (segment (start 120.8 79.74) (end 120.74 79.74) (width 0.25) (layer "F.Cu") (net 18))
 (segment (start 129.5 52.5) (end 118.25 63.75) (width 0.25) (layer "F.Cu") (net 18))
 (segment (start 120.74 79.74) (end 120.5 79.5) (width 0.25) (layer "F.Cu") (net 18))
 (segment (start 118.25 77.19) (end 120.8 79.74) (width 0.25) (layer "F.Cu") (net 18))
 (segment (start 133.276 52.5) (end 129.5 52.5) (width 0.25) (layer "F.Cu") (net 18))
 (segment (start 118.25 63.75) (end 118.25 77.19) (width 0.25) (layer "F.Cu") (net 18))
 (segment (start 136.576 49.2) (end 133.276 52.5) (width 0.25) (layer "F.Cu") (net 18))
 (segment (start 123.75028 63) (end 120.25 63) (width 0.25) (layer "F.Cu") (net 19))
 (segment (start 131.95 60.05) (end 130.2 60.05) (width 0.25) (layer "F.Cu") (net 19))
 (segment (start 119.25 64) (end 119.25 75.65) (width 0.25) (layer "F.Cu") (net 19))
 (segment (start 130.2 60.05) (end 127.15 63.1) (width 0.25) (layer "F.Cu") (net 19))
 (segment (start 124.6 63.84972) (end 123.75028 63) (width 0.25) (layer "F.Cu") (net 19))
 (segment (start 139.116 49.2) (end 139.116 52.884) (width 0.25) (layer "F.Cu") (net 19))
 (segment (start 120.25 63) (end 119.25 64) (width 0.25) (layer "F.Cu") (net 19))
 (segment (start 127.15 65.14028) (end 126.29028 66) (width 0.25) (layer "F.Cu") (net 19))
 (segment (start 139.116 52.884) (end 131.95 60.05) (width 0.25) (layer "F.Cu") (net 19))
 (segment (start 124.6 65.123604) (end 124.6 63.84972) (width 0.25) (layer "F.Cu") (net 19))
 (segment (start 125.476396 66) (end 124.6 65.123604) (width 0.25) (layer "F.Cu") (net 19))
 (segment (start 126.29028 66) (end 125.476396 66) (width 0.25) (layer "F.Cu") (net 19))
 (segment (start 127.15 63.1) (end 127.15 65.14028) (width 0.25) (layer "F.Cu") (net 19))
 (segment (start 119.25 75.65) (end 123.34 79.74) (width 0.25) (layer "F.Cu") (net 19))
 (segment (start 153.34 49.2) (end 157.5 53.36) (width 0.25) (layer "F.Cu") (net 24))
 (segment (start 157.5 53.36) (end 157.5 67.5) (width 0.25) (layer "F.Cu") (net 24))
 (segment (start 163.5 54.28) (end 163.5 67.5) (width 0.25) (layer "F.Cu") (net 26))
 (segment (start 158.42 49.2) (end 163.5 54.28) (width 0.25) (layer "F.Cu") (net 26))
 (segment (start 123.34 65.59) (end 126.9 69.15) (width 0.25) (layer "F.Cu") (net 22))
 (segment (start 156 79.75) (end 156.75 80.5) (width 0.25) (layer "F.Cu") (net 22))
 (segment (start 159.75 80.5) (end 162 78.25) (width 0.25) (layer "F.Cu") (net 22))
 (segment (start 157.15 48.4) (end 156.5 47.75) (width 0.25) (layer "F.Cu") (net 22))
 (segment (start 162 78.25) (end 162 54.75) (width 0.25) (layer "F.Cu") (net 22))
 (segment (start 154.25 74.3) (end 156 76.05) (width 0.25) (layer "F.Cu") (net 22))
 (segment (start 157.15 49.9) (end 157.15 48.4) (width 0.25) (layer "F.Cu") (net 22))
 (segment (start 126.9 69.15) (end 126.9 70.75) (width 0.25) (layer "F.Cu") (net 22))
 (segment (start 156.5 47.75) (end 149.71 47.75) (width 0.25) (layer "F.Cu") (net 22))
 (segment (start 149.71 47.75) (end 148.26 49.2) (width 0.25) (layer "F.Cu") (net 22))
 (segment (start 156 76.05) (end 156 79.75) (width 0.25) (layer "F.Cu") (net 22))
 (segment (start 162 54.75) (end 157.15 49.9) (width 0.25) (layer "F.Cu") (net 22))
 (segment (start 123.34 64.5) (end 123.34 65.59) (width 0.25) (layer "F.Cu") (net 22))
 (segment (start 130.45 74.3) (end 154.25 74.3) (width 0.25) (layer "F.Cu") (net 22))
 (segment (start 126.9 70.75) (end 130.45 74.3) (width 0.25) (layer "F.Cu") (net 22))
 (segment (start 156.75 80.5) (end 159.75 80.5) (width 0.25) (layer "F.Cu") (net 22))
 (segment (start 154.95 67.5) (end 155 67.5) (width 0.25) (layer "F.Cu") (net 23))
 (segment (start 154.5 52.9) (end 150.8 49.2) (width 0.25) (layer "F.Cu") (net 23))
 (segment (start 154.5 67.5) (end 154.5 52.9) (width 0.25) (layer "F.Cu") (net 23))
 (segment (start 155.88 49.88) (end 158.75 52.75) (width 0.25) (layer "F.Cu") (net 25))
 (segment (start 158.75 65.75) (end 160.5 67.5) (width 0.25) (layer "F.Cu") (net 25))
 (segment (start 158.75 52.75) (end 158.75 65.75) (width 0.25) (layer "F.Cu") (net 25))
 (segment (start 155.88 49.2) (end 155.88 49.88) (width 0.25) (layer "F.Cu") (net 25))
 (segment (start 145.54 97.46) (end 145.5 97.5) (width 0.25) (layer "F.Cu") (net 7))
 (segment (start 145.72 97.46) (end 145.54 97.46) (width 0.25) (layer "F.Cu") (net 7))
 (segment (start 125 71.875) (end 125 68.7) (width 0.25) (layer "F.Cu") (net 32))
 (segment (start 163.5 77.66) (end 163.5 78.75) (width 0.25) (layer "F.Cu") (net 32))
 (segment (start 157.75 84.5) (end 135.75 84.5) (width 0.25) (layer "F.Cu") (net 32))
 (segment (start 135.75 84.5) (end 132.25 81) (width 0.25) (layer "F.Cu") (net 32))
 (segment (start 125 68.7) (end 120.8 64.5) (width 0.25) (layer "F.Cu") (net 32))
 (segment (start 132.25 81) (end 132.25 79.125) (width 0.25) (layer "F.Cu") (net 32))
 (segment (start 132.25 79.125) (end 125 71.875) (width 0.25) (layer "F.Cu") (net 32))
 (segment (start 163.5 78.75) (end 157.75 84.5) (width 0.25) (layer "F.Cu") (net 32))
 (segment (start 134 71.5) (end 154.25 71.5) (width 0.25) (layer "F.Cu") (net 30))
 (segment (start 154.25 71.5) (end 157.5 74.75) (width 0.25) (layer "F.Cu") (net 30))
 (segment (start 157.5 74.75) (end 157.5 77.66) (width 0.25) (layer "F.Cu") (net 30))
 (segment (start 130.96 68.46) (end 134 71.5) (width 0.25) (layer "F.Cu") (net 30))
 (segment (start 130.96 64.5) (end 130.96 68.46) (width 0.25) (layer "F.Cu") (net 30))
 (segment (start 132.25 63.45) (end 132.25 65.85) (width 0.25) (layer "F.Cu") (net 31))
 (segment (start 132.25 65.85) (end 136.3 69.9) (width 0.25) (layer "F.Cu") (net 31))
 (segment (start 128.42 63.58) (end 129.35 62.65) (width 0.25) (layer "F.Cu") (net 31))
 (segment (start 155.4 69.9) (end 160.5 75) (width 0.25) (layer "F.Cu") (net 31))
 (segment (start 128.42 64.5) (end 128.42 63.58) (width 0.25) (layer "F.Cu") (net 31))
 (segment (start 136.3 69.9) (end 155.4 69.9) (width 0.25) (layer "F.Cu") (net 31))
 (segment (start 131.45 62.65) (end 132.25 63.45) (width 0.25) (layer "F.Cu") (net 31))
 (segment (start 160.5 75) (end 160.5 77.66) (width 0.25) (layer "F.Cu") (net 31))
 (segment (start 129.35 62.65) (end 131.45 62.65) (width 0.25) (layer "F.Cu") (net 31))
 (segment (start 153.5 83.5) (end 154.5 82.5) (width 0.25) (layer "F.Cu") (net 29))
 (segment (start 133.5 79.74) (end 137.26 83.5) (width 0.25) (layer "F.Cu") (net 29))
 (segment (start 154.5 82.5) (end 154.5 77.66) (width 0.25) (layer "F.Cu") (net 29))
 (segment (start 137.26 83.5) (end 153.5 83.5) (width 0.25) (layer "F.Cu") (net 29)))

